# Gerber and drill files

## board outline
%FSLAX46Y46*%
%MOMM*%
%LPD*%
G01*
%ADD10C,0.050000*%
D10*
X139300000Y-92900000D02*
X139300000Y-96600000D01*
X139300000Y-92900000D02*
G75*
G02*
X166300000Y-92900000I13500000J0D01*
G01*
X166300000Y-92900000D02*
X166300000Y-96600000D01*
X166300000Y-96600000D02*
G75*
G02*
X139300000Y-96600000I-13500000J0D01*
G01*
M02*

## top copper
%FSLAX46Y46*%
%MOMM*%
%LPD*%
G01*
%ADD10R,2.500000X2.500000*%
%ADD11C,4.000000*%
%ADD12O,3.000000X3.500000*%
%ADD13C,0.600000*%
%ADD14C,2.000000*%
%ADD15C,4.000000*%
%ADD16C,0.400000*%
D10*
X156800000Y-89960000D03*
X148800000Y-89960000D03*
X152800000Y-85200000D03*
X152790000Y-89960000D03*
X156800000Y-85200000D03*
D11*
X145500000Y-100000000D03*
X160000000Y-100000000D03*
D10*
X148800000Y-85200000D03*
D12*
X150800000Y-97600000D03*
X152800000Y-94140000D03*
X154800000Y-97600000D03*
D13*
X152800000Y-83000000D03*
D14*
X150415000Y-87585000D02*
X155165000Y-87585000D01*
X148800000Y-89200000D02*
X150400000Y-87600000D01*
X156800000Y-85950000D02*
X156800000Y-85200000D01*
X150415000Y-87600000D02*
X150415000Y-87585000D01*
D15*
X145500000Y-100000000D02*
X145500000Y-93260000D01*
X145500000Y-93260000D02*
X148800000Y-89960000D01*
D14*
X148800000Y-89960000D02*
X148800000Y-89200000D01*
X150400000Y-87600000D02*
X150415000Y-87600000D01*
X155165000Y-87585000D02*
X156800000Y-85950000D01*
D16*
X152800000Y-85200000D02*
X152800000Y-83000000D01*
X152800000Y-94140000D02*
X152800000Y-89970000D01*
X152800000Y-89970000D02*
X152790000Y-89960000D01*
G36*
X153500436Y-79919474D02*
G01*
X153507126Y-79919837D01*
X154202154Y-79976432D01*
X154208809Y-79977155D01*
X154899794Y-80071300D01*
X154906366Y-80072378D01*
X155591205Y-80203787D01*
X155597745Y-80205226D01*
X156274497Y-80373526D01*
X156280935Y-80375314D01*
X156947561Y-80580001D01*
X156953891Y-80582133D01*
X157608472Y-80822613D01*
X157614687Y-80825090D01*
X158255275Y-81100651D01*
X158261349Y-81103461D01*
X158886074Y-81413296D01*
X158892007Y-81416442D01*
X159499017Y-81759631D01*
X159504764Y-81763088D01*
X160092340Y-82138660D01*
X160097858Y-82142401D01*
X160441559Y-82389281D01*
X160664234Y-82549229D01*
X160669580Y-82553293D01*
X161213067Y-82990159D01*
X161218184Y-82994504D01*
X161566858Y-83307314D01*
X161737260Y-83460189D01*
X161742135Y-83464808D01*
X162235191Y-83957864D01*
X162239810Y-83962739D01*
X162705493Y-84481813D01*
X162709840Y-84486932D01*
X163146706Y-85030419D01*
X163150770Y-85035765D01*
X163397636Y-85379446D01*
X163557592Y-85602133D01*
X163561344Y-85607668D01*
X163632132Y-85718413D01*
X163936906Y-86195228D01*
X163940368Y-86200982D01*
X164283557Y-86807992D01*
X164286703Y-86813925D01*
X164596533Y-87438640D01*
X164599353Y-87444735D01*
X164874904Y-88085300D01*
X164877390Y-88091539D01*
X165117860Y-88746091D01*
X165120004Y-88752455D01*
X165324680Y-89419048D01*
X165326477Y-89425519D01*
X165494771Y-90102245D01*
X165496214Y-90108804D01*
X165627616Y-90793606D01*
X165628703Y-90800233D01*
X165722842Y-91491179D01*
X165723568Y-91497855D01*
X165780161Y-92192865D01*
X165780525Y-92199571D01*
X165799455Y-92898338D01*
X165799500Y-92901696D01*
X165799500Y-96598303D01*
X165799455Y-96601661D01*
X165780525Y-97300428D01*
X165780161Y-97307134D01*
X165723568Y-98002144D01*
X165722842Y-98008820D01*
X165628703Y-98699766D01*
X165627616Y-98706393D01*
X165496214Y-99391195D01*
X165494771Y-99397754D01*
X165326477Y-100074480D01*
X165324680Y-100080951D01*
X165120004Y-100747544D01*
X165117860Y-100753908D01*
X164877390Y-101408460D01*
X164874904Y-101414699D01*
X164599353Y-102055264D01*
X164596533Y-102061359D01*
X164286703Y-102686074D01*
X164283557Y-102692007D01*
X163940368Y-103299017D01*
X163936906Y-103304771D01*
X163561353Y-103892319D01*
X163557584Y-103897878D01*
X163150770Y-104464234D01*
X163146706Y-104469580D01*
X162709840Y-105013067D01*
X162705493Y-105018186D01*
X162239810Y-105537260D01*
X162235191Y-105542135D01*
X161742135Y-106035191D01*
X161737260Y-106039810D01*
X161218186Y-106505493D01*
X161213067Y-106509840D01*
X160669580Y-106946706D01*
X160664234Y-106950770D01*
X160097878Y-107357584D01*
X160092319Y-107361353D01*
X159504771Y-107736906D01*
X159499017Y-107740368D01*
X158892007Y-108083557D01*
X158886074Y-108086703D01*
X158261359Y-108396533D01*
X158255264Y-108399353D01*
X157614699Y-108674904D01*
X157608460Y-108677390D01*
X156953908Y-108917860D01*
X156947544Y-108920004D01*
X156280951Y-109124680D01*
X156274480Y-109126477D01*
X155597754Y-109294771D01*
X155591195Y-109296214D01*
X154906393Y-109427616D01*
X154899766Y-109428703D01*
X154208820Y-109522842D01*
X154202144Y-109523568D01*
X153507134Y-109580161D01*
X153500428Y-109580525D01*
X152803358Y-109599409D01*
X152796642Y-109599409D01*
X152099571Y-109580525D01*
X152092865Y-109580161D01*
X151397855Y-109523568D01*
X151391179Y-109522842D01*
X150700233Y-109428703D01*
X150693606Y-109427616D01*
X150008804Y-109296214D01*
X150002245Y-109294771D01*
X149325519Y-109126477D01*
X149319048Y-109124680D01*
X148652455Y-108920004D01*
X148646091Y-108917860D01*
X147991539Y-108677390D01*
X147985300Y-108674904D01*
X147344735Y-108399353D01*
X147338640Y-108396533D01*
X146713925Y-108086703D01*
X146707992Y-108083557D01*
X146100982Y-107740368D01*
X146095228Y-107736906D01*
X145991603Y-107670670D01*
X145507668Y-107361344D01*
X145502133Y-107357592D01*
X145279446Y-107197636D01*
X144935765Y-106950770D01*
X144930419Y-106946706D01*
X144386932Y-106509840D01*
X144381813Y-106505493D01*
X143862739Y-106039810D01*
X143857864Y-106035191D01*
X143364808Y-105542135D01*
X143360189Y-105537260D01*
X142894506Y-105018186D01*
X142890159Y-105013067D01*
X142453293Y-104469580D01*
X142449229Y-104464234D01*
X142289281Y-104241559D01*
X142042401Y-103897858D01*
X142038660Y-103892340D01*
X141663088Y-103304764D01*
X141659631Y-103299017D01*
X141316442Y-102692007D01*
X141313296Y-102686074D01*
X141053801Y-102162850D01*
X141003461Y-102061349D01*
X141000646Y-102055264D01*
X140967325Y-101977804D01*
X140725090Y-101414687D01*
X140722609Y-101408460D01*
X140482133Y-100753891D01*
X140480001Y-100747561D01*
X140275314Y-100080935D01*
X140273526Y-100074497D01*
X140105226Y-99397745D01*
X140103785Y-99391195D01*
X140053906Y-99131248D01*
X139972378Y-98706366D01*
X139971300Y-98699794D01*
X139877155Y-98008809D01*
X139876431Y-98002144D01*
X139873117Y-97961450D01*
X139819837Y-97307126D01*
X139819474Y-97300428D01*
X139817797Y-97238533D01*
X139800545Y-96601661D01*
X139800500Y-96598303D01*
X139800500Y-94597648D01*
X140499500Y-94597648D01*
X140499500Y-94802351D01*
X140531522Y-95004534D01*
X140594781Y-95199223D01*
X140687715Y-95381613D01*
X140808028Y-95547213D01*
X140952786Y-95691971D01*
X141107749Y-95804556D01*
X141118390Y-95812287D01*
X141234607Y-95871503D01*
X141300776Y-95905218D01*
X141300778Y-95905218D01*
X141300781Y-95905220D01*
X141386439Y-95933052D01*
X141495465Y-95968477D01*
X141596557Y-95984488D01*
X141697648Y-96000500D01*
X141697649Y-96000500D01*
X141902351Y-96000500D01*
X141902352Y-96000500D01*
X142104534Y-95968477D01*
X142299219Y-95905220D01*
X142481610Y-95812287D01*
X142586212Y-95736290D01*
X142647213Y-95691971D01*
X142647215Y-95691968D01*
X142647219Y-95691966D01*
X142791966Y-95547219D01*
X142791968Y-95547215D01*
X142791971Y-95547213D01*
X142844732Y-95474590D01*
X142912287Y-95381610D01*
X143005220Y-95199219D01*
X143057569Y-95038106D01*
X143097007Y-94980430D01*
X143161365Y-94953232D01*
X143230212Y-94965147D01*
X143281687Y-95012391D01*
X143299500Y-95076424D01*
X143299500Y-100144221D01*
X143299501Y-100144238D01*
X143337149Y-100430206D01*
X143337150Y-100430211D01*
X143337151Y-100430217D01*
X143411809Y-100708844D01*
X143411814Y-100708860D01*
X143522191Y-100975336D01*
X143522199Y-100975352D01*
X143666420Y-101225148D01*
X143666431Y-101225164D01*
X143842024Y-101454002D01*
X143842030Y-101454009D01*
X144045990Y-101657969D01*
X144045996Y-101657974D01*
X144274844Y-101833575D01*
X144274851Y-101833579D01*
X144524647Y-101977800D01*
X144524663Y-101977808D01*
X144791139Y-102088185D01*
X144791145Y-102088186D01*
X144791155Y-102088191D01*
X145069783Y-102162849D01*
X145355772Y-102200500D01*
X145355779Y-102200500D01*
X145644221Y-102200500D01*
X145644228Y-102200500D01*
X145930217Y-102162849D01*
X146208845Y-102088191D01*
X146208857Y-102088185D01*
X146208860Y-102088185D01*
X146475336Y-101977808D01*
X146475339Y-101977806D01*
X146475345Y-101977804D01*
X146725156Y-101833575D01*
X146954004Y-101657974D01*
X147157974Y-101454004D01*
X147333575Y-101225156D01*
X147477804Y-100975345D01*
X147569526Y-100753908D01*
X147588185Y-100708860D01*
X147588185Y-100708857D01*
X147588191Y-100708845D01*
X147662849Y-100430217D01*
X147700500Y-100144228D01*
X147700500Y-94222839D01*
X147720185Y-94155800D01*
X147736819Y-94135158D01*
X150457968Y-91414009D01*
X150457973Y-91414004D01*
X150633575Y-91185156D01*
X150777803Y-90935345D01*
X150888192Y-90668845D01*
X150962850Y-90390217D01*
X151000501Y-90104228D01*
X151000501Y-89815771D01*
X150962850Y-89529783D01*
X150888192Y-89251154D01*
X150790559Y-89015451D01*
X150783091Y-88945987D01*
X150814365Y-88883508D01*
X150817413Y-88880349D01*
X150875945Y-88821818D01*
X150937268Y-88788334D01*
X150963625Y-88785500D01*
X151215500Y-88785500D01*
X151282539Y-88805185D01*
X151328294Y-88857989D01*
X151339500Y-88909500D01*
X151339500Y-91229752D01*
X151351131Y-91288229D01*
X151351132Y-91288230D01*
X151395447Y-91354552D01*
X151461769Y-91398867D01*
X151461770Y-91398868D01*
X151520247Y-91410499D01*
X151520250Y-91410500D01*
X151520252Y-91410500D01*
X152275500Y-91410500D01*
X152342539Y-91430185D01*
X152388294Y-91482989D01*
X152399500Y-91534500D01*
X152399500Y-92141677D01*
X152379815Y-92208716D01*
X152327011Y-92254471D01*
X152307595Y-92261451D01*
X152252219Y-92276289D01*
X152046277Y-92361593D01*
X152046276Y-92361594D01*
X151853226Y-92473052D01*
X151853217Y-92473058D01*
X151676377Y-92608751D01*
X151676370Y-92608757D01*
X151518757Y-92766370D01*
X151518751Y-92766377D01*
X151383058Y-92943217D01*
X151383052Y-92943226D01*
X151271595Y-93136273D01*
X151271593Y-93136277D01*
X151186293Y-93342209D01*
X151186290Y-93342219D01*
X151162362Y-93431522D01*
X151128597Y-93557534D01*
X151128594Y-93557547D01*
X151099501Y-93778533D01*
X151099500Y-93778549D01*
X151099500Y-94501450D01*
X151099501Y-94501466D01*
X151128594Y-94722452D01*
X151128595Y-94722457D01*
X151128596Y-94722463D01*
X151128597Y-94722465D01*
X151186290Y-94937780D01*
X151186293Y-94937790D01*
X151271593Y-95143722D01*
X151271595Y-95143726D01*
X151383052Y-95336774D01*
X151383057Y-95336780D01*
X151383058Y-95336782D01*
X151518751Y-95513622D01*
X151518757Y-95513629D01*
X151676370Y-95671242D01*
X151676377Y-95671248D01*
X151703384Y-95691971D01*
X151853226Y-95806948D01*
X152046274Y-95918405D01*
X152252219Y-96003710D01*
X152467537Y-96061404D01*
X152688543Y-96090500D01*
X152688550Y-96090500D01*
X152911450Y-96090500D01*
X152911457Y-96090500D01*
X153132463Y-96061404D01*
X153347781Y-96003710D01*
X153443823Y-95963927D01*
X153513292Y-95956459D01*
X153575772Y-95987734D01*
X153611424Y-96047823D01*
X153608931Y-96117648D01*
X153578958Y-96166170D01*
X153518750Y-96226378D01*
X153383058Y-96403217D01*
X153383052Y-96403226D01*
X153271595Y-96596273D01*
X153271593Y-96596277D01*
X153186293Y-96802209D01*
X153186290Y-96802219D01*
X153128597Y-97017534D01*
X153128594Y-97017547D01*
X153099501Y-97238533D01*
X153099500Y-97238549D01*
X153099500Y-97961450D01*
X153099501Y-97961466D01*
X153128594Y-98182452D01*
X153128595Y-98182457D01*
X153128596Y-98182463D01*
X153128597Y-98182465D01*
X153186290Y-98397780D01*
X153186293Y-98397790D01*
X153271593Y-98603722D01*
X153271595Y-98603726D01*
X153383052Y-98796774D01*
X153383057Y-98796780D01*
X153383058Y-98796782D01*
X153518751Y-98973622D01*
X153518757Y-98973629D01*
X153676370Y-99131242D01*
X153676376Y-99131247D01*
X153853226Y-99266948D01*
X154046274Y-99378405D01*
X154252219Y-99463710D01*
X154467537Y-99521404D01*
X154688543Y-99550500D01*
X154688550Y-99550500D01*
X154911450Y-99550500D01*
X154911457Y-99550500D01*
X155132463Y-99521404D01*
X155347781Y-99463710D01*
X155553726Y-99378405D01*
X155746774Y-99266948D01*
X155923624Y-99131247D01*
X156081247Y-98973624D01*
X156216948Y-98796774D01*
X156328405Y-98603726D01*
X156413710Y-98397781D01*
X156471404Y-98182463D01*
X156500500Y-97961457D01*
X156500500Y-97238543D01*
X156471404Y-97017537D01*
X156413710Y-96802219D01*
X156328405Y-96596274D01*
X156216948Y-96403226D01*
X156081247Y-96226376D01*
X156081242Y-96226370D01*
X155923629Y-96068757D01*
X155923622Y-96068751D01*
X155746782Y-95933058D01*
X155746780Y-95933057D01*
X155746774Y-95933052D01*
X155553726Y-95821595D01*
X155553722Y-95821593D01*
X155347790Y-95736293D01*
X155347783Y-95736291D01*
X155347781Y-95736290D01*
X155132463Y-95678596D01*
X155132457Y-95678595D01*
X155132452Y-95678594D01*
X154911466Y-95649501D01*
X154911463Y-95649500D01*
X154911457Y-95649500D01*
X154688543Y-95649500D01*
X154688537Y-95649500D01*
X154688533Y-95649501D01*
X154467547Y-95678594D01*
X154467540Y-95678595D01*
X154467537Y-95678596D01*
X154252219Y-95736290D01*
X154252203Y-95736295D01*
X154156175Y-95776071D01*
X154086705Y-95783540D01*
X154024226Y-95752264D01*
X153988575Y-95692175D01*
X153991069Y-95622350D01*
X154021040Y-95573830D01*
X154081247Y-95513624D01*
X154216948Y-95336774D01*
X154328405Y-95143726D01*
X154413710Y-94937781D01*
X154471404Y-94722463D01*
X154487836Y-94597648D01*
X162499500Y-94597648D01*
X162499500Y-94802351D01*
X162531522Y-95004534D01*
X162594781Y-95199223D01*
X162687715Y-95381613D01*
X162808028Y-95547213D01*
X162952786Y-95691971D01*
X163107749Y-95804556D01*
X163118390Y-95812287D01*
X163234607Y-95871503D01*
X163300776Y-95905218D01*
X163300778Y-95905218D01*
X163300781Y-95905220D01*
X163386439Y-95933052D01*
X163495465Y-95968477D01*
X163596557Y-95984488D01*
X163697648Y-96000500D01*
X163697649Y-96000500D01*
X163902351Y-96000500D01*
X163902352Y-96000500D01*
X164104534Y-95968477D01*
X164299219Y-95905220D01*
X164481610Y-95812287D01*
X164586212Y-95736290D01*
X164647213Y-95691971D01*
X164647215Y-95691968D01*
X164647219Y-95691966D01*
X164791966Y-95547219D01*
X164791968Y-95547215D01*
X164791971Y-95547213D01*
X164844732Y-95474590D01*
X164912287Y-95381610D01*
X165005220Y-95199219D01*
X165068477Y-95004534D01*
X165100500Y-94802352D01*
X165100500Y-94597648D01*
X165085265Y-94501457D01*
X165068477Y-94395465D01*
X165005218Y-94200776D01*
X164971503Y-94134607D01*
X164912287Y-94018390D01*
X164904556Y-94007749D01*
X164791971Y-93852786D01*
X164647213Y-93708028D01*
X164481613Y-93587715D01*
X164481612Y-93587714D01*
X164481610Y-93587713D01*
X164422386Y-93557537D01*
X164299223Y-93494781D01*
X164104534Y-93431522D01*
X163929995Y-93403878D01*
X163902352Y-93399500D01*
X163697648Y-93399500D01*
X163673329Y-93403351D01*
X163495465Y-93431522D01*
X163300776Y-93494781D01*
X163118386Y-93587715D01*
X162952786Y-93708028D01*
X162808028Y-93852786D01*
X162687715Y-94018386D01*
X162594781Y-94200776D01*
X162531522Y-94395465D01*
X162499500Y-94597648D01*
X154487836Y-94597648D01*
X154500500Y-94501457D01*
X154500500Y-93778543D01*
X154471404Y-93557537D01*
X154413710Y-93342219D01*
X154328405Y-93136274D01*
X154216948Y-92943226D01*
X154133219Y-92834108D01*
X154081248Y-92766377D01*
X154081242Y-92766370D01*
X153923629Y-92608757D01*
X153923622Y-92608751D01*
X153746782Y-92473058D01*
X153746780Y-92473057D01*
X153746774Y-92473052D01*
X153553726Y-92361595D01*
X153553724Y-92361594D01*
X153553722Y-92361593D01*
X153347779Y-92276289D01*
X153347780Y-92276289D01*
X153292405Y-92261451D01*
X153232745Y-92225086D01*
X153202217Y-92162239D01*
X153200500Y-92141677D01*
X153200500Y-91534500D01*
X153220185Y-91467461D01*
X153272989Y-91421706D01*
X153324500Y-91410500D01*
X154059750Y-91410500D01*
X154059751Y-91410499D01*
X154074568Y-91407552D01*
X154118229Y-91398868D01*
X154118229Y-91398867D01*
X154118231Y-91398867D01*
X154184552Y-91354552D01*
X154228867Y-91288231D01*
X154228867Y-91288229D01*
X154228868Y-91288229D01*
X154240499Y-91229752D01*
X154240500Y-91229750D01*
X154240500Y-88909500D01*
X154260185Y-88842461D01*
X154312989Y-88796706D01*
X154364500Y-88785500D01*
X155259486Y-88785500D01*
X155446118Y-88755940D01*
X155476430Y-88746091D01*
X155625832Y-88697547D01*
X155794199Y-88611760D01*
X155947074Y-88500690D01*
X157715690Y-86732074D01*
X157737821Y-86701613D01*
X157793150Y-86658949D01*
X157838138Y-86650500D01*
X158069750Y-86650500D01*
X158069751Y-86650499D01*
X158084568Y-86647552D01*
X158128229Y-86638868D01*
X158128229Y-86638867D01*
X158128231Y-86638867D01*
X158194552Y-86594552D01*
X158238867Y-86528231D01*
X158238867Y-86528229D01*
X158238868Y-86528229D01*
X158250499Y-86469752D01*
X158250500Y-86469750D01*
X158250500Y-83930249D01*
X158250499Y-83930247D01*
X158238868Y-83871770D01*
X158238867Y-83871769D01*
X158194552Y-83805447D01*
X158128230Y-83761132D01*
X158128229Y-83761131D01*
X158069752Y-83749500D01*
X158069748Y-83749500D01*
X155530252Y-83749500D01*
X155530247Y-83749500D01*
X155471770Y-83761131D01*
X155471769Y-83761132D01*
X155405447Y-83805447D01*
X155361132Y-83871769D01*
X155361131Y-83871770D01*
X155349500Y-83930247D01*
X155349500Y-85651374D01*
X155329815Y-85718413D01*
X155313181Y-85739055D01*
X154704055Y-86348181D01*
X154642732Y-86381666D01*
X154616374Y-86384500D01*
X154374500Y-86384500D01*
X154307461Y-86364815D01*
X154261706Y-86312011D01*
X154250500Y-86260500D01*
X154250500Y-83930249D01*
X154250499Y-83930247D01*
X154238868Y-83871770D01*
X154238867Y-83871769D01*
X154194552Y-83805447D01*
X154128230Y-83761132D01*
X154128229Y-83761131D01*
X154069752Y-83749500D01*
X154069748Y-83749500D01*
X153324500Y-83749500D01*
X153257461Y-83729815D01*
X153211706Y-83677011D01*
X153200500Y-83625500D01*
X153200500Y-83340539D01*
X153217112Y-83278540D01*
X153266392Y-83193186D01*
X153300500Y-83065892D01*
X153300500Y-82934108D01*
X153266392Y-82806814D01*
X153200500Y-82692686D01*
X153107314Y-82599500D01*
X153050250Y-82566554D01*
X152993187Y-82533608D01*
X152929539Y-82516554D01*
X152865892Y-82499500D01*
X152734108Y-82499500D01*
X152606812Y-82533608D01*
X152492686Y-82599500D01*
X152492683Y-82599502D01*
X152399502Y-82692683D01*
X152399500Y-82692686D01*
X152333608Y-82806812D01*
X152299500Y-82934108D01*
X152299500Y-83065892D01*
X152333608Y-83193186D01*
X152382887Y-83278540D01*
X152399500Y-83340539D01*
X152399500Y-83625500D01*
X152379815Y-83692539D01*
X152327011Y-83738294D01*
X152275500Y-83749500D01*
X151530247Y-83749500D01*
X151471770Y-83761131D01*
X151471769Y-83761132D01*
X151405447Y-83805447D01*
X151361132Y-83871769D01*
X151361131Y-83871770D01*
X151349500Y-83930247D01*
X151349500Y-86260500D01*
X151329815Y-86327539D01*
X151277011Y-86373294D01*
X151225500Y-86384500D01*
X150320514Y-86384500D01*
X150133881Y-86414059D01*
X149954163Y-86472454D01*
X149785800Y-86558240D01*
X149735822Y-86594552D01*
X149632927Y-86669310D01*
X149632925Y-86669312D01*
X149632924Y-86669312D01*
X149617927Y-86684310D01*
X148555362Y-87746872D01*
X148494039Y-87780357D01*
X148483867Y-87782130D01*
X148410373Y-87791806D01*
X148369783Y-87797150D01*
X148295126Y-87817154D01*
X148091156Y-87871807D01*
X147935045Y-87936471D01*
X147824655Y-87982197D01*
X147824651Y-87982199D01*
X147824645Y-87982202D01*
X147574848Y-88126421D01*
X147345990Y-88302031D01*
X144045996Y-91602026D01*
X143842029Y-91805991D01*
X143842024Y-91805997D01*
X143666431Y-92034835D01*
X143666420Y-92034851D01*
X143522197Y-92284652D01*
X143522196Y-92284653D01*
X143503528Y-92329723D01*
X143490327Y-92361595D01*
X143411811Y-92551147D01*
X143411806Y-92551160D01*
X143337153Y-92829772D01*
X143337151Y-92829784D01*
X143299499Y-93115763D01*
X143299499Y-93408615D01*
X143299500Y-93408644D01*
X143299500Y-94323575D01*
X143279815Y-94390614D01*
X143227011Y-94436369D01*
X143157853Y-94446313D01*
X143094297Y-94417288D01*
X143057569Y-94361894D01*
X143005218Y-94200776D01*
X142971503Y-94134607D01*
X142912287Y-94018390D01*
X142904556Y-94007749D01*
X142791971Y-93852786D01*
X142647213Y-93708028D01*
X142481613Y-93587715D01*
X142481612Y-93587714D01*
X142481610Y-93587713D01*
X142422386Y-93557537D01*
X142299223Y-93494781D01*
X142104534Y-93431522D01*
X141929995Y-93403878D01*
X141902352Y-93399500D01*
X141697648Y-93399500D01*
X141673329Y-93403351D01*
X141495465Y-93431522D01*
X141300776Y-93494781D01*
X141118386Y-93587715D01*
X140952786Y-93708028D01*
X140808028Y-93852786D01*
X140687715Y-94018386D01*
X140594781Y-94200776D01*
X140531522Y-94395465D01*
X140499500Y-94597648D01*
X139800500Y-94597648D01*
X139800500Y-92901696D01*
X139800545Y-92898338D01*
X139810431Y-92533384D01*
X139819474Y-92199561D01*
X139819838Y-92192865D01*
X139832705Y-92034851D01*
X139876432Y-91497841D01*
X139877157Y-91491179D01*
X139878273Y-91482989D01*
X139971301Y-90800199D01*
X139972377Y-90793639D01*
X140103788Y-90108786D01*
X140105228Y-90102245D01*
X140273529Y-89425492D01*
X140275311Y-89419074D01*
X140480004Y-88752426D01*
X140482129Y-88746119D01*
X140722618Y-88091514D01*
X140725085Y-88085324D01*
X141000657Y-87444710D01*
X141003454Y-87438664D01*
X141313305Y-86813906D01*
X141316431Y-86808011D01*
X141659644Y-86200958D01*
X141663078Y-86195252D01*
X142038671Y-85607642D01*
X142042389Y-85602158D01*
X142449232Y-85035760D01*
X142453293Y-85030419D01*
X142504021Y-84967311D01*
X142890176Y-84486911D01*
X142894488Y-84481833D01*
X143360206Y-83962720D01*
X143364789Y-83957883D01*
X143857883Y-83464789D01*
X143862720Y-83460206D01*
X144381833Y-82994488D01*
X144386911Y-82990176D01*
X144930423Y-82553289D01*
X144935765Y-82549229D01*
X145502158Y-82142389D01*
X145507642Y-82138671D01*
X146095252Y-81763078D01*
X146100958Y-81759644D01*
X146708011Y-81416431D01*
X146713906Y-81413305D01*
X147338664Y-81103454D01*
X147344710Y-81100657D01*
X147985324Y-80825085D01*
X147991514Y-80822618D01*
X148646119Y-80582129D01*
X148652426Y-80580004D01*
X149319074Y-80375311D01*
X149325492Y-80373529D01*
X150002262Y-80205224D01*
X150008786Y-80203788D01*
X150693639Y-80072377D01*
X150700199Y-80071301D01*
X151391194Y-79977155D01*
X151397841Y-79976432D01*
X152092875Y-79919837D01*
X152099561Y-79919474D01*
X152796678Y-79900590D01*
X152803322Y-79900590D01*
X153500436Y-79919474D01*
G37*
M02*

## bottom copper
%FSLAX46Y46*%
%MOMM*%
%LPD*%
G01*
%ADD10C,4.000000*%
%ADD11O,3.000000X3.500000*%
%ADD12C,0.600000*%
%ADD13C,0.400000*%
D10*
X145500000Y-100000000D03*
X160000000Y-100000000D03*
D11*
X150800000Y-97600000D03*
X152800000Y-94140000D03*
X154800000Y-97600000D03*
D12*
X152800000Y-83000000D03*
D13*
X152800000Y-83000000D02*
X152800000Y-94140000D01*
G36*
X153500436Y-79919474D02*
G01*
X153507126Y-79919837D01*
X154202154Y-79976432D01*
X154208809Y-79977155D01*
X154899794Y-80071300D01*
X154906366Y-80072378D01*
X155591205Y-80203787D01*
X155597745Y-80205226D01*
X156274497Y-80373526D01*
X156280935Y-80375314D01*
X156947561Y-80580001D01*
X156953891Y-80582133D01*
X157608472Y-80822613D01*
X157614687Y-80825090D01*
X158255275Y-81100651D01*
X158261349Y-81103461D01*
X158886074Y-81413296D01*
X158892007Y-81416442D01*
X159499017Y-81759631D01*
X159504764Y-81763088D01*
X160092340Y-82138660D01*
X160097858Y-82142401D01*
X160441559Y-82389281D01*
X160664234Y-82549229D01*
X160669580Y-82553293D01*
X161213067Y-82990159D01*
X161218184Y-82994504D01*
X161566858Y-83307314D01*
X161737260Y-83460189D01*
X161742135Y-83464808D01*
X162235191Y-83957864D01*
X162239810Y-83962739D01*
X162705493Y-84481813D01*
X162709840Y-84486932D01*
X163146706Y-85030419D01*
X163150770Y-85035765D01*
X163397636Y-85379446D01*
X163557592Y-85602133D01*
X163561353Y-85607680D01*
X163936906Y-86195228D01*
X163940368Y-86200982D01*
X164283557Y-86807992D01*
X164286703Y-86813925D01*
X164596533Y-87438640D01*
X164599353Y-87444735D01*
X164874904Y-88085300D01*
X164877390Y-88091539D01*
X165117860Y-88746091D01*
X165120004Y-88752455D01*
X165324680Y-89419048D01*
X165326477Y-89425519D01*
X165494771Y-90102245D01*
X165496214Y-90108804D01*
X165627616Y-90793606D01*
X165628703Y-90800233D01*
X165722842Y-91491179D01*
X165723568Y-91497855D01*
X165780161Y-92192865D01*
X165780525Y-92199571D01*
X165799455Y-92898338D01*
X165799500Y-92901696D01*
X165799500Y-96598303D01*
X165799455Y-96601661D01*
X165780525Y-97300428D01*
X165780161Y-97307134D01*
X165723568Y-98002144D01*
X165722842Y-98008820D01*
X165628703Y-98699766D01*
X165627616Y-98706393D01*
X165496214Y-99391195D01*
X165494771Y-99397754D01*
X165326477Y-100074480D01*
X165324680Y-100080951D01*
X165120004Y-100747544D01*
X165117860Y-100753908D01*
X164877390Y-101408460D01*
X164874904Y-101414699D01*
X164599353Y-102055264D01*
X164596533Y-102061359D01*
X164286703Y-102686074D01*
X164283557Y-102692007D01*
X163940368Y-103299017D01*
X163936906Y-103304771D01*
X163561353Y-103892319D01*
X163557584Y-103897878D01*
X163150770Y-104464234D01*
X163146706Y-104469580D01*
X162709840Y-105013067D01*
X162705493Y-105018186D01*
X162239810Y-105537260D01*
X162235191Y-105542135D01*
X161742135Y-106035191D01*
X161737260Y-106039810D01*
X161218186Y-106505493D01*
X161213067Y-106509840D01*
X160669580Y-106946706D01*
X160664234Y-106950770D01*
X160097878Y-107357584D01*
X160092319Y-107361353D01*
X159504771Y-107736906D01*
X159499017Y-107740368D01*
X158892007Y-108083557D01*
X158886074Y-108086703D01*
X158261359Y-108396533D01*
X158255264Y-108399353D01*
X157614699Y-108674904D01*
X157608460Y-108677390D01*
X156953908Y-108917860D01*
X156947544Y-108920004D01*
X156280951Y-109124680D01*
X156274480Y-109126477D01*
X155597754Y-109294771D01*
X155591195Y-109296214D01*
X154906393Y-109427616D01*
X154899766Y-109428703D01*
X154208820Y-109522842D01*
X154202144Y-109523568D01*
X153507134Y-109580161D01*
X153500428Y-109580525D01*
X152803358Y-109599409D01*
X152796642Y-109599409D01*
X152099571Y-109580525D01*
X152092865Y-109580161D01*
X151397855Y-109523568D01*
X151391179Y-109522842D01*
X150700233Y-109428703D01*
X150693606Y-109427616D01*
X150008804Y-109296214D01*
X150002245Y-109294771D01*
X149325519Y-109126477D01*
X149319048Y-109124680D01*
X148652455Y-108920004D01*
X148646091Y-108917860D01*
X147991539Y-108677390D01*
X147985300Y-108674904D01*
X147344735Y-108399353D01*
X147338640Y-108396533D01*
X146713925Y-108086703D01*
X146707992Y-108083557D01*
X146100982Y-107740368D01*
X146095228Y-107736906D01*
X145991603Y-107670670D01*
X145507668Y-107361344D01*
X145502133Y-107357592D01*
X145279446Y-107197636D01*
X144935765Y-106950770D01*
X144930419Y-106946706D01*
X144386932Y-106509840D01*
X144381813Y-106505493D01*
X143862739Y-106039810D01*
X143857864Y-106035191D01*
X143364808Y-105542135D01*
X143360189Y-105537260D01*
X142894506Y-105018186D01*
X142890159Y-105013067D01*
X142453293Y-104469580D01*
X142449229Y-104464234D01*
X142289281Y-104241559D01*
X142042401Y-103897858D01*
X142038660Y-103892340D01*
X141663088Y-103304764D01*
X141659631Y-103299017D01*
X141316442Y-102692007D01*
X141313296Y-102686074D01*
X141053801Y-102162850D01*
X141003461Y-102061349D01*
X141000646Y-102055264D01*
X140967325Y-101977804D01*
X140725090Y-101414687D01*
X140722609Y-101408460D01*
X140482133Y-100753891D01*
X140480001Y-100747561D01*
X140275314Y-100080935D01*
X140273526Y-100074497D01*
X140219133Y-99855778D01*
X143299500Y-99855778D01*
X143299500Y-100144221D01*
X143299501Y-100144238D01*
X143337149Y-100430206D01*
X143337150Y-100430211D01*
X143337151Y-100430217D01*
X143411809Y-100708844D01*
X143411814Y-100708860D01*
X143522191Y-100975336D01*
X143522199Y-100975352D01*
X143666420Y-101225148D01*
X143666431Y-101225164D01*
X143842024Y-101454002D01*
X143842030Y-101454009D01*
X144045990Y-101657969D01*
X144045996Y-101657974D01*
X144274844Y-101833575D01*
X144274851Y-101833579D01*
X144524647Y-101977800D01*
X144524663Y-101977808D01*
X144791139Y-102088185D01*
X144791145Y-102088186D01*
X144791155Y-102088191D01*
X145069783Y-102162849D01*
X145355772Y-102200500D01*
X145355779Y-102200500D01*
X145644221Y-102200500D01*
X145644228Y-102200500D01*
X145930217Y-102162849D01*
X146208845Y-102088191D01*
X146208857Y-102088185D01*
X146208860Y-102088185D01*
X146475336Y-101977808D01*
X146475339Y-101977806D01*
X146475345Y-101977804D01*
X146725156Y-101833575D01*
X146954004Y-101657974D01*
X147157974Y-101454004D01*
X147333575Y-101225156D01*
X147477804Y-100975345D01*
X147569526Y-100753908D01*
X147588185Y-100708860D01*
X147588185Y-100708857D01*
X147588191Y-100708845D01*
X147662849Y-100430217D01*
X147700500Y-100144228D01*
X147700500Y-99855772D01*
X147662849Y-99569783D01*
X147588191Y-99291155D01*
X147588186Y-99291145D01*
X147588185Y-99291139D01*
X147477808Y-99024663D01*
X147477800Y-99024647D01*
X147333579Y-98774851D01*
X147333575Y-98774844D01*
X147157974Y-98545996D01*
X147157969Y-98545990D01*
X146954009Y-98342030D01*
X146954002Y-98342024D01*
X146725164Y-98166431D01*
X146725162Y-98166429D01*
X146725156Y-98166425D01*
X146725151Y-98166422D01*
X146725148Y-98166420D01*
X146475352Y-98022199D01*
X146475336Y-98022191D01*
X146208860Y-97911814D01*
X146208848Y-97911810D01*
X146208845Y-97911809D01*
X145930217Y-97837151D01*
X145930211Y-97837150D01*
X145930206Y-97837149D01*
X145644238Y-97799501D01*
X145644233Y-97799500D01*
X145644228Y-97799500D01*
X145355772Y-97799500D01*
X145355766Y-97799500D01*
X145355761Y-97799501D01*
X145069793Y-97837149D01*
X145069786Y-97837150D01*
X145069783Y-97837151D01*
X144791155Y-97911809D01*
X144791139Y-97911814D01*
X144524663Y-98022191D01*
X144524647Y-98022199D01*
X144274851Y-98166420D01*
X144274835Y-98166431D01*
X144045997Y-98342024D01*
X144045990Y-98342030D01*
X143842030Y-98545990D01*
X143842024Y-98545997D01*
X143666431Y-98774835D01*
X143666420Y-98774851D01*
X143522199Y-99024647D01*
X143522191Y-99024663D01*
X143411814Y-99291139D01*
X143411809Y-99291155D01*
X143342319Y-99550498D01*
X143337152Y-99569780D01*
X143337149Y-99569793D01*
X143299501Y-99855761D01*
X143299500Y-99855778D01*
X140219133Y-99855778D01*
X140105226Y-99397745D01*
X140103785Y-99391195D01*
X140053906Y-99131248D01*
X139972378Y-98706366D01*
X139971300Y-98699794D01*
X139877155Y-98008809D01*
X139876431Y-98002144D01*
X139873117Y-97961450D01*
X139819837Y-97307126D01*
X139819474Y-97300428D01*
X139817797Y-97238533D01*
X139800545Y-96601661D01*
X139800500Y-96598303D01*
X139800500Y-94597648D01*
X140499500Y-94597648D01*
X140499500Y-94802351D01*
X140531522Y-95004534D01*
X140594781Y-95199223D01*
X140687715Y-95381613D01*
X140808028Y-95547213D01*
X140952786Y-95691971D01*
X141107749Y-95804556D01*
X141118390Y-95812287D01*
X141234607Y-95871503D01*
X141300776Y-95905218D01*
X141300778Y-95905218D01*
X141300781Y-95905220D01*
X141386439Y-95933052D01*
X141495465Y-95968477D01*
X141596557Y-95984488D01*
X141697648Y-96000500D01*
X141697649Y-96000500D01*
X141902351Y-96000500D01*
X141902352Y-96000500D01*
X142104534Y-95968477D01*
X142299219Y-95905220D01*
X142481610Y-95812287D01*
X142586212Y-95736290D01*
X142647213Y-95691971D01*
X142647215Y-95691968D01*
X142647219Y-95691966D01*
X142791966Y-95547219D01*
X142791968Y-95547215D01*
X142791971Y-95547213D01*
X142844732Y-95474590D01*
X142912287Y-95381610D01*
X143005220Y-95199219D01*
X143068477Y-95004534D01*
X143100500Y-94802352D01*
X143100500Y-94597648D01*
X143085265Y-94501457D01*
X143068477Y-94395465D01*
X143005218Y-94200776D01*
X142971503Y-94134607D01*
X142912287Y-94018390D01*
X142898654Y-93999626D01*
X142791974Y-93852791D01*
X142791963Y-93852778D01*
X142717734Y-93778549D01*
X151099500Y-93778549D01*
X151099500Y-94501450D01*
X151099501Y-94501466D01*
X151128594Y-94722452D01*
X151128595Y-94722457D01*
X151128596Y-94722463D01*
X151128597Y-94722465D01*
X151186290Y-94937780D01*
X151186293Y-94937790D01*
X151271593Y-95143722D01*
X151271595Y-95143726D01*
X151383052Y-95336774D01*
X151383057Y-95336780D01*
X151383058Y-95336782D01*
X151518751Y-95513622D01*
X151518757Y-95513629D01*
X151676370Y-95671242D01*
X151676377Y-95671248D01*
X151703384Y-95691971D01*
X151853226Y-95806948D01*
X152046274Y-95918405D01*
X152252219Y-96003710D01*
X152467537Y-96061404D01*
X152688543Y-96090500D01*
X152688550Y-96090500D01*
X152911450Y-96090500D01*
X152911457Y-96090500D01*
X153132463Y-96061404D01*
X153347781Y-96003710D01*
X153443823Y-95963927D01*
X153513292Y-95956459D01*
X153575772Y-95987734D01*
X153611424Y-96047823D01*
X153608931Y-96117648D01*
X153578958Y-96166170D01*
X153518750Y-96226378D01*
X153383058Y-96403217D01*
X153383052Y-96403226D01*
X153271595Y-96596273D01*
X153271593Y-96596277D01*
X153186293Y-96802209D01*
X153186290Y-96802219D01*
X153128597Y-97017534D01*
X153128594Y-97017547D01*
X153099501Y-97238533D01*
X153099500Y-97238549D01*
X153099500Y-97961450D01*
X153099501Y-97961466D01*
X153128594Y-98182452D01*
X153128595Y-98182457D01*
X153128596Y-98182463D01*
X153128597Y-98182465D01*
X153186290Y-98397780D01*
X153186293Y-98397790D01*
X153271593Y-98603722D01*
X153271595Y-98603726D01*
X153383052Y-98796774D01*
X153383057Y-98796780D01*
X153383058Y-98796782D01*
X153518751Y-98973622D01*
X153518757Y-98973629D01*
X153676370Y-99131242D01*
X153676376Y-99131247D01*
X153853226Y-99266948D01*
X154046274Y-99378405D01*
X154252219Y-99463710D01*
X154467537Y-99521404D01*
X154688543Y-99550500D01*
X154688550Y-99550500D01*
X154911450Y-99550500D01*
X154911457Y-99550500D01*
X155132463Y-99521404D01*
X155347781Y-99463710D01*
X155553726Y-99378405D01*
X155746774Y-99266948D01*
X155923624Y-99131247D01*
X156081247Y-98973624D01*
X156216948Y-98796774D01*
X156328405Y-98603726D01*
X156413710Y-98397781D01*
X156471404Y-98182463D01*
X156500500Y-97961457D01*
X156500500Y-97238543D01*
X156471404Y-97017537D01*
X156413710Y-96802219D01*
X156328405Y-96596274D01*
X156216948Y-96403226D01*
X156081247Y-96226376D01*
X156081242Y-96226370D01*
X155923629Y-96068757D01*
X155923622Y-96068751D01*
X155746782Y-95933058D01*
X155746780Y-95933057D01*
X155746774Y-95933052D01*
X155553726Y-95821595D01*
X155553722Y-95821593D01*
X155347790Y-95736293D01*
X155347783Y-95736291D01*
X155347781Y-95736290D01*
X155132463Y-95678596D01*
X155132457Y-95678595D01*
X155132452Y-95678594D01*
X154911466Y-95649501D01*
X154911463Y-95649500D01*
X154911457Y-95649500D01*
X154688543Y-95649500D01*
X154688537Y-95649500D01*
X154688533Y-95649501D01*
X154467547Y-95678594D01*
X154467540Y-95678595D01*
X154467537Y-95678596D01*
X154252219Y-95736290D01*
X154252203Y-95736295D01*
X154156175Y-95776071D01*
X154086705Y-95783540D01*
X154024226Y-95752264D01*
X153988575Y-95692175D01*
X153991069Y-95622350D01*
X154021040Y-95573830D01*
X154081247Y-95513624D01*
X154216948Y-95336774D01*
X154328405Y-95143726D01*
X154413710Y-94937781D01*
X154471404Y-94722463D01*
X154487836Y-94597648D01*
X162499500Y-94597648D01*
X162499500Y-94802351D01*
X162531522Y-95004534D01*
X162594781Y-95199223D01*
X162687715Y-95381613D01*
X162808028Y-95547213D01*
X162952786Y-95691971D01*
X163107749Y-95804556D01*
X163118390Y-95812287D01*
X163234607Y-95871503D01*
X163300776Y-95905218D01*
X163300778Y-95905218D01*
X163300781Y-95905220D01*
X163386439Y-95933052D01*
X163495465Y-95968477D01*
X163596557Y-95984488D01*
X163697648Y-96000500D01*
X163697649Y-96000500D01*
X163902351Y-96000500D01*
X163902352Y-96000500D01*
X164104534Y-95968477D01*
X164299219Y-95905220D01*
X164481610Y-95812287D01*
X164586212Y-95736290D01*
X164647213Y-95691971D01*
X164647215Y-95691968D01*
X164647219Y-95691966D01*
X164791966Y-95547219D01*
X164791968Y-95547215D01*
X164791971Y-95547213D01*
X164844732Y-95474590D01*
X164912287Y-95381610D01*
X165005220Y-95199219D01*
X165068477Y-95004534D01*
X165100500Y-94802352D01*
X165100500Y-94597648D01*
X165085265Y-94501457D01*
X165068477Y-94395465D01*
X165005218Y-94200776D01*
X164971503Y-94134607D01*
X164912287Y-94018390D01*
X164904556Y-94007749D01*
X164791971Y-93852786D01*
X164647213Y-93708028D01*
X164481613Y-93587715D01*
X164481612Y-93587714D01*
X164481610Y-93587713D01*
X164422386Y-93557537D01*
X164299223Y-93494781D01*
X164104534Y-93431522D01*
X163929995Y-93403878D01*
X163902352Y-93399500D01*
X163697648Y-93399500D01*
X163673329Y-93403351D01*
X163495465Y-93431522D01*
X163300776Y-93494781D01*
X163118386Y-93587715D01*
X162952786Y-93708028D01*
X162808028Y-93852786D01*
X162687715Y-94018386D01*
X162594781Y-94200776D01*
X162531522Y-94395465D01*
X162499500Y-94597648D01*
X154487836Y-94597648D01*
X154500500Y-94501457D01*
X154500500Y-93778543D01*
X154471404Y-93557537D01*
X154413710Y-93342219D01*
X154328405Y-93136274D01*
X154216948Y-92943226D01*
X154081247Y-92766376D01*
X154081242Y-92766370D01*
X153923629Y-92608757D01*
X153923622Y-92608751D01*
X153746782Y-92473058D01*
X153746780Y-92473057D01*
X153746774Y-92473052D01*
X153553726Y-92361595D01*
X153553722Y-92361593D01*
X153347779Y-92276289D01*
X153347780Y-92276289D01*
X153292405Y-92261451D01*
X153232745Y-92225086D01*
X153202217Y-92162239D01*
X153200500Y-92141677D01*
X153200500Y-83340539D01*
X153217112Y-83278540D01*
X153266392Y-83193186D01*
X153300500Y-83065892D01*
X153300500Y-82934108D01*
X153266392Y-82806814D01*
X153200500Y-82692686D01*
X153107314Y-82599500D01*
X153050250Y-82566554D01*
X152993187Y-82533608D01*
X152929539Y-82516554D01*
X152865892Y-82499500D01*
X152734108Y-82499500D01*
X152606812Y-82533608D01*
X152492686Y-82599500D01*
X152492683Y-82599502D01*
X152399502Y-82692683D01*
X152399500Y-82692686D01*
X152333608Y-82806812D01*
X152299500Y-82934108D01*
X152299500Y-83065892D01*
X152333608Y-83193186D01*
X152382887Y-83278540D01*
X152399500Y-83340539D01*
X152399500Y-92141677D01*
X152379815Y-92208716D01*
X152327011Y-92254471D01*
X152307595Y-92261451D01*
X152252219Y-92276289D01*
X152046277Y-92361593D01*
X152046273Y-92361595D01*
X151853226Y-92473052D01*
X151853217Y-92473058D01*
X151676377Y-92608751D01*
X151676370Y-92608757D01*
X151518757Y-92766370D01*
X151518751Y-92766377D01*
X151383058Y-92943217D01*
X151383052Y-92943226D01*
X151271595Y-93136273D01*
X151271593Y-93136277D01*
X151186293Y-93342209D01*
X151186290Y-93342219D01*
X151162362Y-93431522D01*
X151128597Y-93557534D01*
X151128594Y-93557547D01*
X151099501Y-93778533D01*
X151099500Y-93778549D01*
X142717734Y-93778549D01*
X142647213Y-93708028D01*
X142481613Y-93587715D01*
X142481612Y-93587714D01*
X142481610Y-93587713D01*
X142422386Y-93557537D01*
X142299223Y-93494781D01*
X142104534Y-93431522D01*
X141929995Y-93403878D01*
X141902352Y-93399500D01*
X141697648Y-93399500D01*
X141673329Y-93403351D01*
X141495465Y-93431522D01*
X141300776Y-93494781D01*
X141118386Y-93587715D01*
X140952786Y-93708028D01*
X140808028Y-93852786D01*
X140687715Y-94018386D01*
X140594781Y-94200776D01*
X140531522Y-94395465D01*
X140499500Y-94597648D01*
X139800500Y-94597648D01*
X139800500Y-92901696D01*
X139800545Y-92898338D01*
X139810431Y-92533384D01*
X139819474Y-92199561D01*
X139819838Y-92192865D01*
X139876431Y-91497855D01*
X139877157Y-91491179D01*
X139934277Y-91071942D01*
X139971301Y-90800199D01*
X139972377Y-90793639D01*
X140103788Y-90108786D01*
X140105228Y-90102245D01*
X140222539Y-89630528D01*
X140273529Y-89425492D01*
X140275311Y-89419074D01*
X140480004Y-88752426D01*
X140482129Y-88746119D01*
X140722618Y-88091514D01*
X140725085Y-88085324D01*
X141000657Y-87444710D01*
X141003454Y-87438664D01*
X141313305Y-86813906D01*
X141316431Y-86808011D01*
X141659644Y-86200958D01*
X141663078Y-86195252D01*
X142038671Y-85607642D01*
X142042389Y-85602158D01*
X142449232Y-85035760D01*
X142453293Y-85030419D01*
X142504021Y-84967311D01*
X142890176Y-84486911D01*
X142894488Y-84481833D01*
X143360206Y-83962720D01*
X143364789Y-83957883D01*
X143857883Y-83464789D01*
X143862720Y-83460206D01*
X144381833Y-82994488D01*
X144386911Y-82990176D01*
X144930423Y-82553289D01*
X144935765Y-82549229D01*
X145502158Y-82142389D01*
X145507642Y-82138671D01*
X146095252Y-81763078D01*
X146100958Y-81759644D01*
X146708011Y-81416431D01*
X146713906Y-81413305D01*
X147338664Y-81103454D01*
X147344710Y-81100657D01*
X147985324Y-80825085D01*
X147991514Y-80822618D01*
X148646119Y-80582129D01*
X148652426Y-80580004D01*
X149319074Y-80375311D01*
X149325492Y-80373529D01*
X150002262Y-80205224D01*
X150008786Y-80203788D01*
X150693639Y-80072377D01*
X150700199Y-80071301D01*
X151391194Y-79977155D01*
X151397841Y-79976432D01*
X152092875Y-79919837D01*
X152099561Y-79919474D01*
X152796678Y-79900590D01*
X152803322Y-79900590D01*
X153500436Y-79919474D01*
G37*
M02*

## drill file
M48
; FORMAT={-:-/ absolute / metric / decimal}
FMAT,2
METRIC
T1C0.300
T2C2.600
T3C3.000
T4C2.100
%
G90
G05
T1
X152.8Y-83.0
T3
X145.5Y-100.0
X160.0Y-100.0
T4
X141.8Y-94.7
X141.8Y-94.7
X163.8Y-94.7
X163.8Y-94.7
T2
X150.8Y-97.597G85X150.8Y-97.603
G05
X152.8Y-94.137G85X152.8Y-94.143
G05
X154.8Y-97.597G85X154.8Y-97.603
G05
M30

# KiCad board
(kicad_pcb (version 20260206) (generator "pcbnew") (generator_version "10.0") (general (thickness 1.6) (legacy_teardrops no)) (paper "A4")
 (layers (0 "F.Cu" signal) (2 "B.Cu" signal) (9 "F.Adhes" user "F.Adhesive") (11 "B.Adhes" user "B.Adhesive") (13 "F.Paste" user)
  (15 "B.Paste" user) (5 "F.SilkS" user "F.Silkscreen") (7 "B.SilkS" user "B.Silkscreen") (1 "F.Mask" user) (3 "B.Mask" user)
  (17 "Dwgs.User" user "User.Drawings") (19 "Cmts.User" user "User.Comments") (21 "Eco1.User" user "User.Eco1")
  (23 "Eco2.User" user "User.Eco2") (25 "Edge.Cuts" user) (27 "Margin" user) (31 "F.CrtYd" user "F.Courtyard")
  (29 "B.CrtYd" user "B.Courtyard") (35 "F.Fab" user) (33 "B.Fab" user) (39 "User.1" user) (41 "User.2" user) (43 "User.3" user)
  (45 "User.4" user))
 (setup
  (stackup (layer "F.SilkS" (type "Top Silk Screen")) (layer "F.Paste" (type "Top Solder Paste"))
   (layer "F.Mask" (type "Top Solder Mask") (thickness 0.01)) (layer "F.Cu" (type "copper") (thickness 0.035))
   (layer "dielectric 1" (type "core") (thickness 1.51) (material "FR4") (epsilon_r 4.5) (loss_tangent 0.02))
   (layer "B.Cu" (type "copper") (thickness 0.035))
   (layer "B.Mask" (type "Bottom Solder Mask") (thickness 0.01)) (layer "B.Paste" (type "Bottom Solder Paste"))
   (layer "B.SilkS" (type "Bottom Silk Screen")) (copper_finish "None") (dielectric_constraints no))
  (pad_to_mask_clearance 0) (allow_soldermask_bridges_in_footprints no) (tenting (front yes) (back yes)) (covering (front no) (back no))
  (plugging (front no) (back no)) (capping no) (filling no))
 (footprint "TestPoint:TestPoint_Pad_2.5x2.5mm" (layer "F.Cu") (at 156.8 89.96)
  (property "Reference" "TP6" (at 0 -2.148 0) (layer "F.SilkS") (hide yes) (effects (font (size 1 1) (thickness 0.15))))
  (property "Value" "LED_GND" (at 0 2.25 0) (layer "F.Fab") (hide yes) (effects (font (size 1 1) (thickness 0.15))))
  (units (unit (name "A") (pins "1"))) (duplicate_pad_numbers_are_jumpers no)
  (pad "1" smd rect (at 0 0) (size 2.5 2.5) (layers "F.Cu" "F.Mask") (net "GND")))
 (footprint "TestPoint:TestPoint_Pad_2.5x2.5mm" (layer "F.Cu") (at 148.8 89.96)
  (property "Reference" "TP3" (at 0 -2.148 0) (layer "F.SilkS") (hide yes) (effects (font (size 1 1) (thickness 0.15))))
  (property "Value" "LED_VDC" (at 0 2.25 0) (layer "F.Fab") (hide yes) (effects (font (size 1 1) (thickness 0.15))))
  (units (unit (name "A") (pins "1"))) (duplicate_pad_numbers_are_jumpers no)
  (pad "1" smd rect (at 0 0) (size 2.5 2.5) (layers "F.Cu" "F.Mask") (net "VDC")))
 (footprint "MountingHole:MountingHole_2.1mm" (layer "F.Cu") (at 163.8 94.7)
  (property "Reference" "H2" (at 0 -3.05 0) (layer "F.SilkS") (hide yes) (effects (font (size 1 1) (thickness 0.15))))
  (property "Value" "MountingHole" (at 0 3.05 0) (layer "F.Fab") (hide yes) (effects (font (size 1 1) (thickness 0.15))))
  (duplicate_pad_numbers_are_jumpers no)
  (pad "" np_thru_hole circle (at 0 0) (size 2.1 2.1) (drill 2.1) (layers "*.Cu" "*.Mask")))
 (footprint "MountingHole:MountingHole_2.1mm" (layer "F.Cu") (at 163.8 94.7)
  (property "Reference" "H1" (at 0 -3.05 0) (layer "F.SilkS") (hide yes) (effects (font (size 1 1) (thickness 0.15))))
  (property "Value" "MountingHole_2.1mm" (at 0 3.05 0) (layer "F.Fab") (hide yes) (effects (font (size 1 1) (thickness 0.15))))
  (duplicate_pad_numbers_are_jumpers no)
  (pad "" np_thru_hole circle (at 0 0) (size 1.6 1.6) (drill 2.1) (layers "*.Cu" "*.Mask")))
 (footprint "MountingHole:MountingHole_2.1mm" (layer "F.Cu") (at 141.8 94.7)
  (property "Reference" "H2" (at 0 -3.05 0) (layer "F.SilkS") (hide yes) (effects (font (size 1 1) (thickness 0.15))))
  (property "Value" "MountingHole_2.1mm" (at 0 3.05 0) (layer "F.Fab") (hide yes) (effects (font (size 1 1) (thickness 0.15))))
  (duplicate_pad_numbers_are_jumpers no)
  (pad "" np_thru_hole circle (at 0 0) (size 1.6 1.6) (drill 2.1) (layers "*.Cu" "*.Mask")))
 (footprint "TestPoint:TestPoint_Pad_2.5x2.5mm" (layer "F.Cu") (at 152.8 85.2)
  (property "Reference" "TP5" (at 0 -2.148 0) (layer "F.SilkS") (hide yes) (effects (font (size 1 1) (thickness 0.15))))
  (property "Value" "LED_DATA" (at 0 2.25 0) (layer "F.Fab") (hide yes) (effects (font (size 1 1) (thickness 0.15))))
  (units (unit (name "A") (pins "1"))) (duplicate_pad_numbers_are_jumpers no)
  (pad "1" smd rect (at 0 0) (size 2.5 2.5) (layers "F.Cu" "F.Mask") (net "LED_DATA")))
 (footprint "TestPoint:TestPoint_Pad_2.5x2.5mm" (layer "F.Cu") (at 152.79 89.96)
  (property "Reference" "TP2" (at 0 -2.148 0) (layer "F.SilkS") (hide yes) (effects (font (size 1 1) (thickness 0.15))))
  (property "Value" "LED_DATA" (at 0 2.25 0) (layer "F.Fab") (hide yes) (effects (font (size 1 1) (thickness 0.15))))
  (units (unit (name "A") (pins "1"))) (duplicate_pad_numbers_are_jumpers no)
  (pad "1" smd rect (at 0 0) (size 2.5 2.5) (layers "F.Cu" "F.Mask") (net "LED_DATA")))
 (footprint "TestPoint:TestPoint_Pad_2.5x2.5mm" (layer "F.Cu") (at 156.8 85.2)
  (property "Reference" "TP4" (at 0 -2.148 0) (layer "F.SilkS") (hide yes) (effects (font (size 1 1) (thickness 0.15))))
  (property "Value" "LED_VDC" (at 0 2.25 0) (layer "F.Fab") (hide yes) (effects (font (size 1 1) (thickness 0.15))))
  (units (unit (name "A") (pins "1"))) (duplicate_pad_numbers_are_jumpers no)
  (pad "1" smd rect (at 0 0) (size 2.5 2.5) (layers "F.Cu" "F.Mask") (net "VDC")))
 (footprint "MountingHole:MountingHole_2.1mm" (layer "F.Cu") (at 141.8 94.7)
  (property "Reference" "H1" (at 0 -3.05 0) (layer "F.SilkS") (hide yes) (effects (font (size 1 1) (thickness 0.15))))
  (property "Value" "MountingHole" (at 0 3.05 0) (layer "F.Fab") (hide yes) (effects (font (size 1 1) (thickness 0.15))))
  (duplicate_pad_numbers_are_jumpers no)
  (pad "" np_thru_hole circle (at 0 0) (size 2.1 2.1) (drill 2.1) (layers "*.Cu" "*.Mask")))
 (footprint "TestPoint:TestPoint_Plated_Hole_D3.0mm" (layer "F.Cu") (at 145.5 100)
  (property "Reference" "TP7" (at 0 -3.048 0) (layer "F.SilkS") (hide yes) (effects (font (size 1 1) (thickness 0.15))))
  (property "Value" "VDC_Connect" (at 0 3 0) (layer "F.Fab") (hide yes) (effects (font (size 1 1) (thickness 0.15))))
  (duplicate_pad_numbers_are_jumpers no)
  (pad "1" thru_hole circle (at 0 0) (size 4 4) (drill 3) (layers "*.Cu" "*.Mask") (remove_unused_layers no) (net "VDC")))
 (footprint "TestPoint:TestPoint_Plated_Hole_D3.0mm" (layer "F.Cu") (at 160 100)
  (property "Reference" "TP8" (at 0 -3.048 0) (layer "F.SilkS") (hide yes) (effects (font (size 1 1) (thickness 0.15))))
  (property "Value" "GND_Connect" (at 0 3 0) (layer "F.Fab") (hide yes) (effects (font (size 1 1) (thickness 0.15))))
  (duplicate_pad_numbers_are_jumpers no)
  (pad "1" thru_hole circle (at 0 0) (size 4 4) (drill 3) (layers "*.Cu" "*.Mask") (remove_unused_layers no) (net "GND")))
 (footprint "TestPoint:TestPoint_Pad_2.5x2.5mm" (layer "F.Cu") (at 148.8 85.2)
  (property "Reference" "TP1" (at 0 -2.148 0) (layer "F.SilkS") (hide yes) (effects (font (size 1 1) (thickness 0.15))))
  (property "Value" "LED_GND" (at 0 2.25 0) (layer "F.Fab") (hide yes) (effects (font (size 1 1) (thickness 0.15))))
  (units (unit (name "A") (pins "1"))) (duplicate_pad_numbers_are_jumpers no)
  (pad "1" smd rect (at 0 0) (size 2.5 2.5) (layers "F.Cu" "F.Mask") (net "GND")))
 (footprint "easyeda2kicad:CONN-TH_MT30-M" (layer "B.Cu") (at 152.8 95.87 -90)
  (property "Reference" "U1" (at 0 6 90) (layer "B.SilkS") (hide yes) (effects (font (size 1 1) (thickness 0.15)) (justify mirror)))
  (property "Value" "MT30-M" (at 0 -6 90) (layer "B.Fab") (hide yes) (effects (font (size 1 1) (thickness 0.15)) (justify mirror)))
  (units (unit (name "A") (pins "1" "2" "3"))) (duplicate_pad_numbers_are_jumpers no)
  (pad "1" thru_hole oval (at 1.73 2 270) (size 3.5 3) (drill oval 2.605075 2.599995) (layers "*.Cu" "*.Mask") (remove_unused_layers no)
   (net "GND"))
  (pad "2" thru_hole oval (at -1.73 0 270) (size 3.5 3) (drill oval 2.605075 2.599995) (layers "*.Cu" "*.Mask") (remove_unused_layers no)
   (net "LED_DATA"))
  (pad "3" thru_hole oval (at 1.73 -2 270) (size 3.5 3) (drill oval 2.605075 2.599995) (layers "*.Cu" "*.Mask") (remove_unused_layers no)
   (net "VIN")))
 (gr_line (start 139.3 92.9) (end 139.3 96.6) (stroke (width 0.05) (type default)) (layer "Edge.Cuts"))
 (gr_arc (start 139.3 92.9) (mid 152.8 79.4) (end 166.3 92.9) (stroke (width 0.05) (type default)) (layer "Edge.Cuts"))
 (gr_line (start 166.3 92.9) (end 166.3 96.6) (stroke (width 0.05) (type default)) (layer "Edge.Cuts"))
 (gr_arc (start 166.3 96.6) (mid 152.8 110.1) (end 139.3 96.6) (stroke (width 0.05) (type default)) (layer "Edge.Cuts"))
 (segment (start 150.415 87.585) (end 155.165 87.585) (width 2) (layer "F.Cu") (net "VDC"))
 (segment (start 148.8 89.2) (end 150.4 87.6) (width 2) (layer "F.Cu") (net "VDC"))
 (segment (start 156.8 85.95) (end 156.8 85.2) (width 2) (layer "F.Cu") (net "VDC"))
 (segment (start 150.415 87.6) (end 150.415 87.585) (width 2) (layer "F.Cu") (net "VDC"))
 (segment (start 145.5 100) (end 145.5 93.26) (width 4) (layer "F.Cu") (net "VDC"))
 (segment (start 145.5 93.26) (end 148.8 89.96) (width 4) (layer "F.Cu") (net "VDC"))
 (segment (start 148.8 89.96) (end 148.8 89.2) (width 2) (layer "F.Cu") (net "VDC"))
 (segment (start 150.4 87.6) (end 150.415 87.6) (width 2) (layer "F.Cu") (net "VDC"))
 (segment (start 155.165 87.585) (end 156.8 85.95) (width 2) (layer "F.Cu") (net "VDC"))
 (segment (start 152.8 85.2) (end 152.8 83) (width 0.4) (layer "F.Cu") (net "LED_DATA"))
 (segment (start 152.8 94.14) (end 152.8 89.97) (width 0.4) (layer "F.Cu") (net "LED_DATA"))
 (segment (start 152.8 89.97) (end 152.79 89.96) (width 0.4) (layer "F.Cu") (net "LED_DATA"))
 (via (at 152.8 83) (size 0.6) (drill 0.3) (layers "F.Cu" "B.Cu") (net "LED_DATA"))
 (segment (start 152.8 83) (end 152.8 94.14) (width 0.4) (layer "B.Cu") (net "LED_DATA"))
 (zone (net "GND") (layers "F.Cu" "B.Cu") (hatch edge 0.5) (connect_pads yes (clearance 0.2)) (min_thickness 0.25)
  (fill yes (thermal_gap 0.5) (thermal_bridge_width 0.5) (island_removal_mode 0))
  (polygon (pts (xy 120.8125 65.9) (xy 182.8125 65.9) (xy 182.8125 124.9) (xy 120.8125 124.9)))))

